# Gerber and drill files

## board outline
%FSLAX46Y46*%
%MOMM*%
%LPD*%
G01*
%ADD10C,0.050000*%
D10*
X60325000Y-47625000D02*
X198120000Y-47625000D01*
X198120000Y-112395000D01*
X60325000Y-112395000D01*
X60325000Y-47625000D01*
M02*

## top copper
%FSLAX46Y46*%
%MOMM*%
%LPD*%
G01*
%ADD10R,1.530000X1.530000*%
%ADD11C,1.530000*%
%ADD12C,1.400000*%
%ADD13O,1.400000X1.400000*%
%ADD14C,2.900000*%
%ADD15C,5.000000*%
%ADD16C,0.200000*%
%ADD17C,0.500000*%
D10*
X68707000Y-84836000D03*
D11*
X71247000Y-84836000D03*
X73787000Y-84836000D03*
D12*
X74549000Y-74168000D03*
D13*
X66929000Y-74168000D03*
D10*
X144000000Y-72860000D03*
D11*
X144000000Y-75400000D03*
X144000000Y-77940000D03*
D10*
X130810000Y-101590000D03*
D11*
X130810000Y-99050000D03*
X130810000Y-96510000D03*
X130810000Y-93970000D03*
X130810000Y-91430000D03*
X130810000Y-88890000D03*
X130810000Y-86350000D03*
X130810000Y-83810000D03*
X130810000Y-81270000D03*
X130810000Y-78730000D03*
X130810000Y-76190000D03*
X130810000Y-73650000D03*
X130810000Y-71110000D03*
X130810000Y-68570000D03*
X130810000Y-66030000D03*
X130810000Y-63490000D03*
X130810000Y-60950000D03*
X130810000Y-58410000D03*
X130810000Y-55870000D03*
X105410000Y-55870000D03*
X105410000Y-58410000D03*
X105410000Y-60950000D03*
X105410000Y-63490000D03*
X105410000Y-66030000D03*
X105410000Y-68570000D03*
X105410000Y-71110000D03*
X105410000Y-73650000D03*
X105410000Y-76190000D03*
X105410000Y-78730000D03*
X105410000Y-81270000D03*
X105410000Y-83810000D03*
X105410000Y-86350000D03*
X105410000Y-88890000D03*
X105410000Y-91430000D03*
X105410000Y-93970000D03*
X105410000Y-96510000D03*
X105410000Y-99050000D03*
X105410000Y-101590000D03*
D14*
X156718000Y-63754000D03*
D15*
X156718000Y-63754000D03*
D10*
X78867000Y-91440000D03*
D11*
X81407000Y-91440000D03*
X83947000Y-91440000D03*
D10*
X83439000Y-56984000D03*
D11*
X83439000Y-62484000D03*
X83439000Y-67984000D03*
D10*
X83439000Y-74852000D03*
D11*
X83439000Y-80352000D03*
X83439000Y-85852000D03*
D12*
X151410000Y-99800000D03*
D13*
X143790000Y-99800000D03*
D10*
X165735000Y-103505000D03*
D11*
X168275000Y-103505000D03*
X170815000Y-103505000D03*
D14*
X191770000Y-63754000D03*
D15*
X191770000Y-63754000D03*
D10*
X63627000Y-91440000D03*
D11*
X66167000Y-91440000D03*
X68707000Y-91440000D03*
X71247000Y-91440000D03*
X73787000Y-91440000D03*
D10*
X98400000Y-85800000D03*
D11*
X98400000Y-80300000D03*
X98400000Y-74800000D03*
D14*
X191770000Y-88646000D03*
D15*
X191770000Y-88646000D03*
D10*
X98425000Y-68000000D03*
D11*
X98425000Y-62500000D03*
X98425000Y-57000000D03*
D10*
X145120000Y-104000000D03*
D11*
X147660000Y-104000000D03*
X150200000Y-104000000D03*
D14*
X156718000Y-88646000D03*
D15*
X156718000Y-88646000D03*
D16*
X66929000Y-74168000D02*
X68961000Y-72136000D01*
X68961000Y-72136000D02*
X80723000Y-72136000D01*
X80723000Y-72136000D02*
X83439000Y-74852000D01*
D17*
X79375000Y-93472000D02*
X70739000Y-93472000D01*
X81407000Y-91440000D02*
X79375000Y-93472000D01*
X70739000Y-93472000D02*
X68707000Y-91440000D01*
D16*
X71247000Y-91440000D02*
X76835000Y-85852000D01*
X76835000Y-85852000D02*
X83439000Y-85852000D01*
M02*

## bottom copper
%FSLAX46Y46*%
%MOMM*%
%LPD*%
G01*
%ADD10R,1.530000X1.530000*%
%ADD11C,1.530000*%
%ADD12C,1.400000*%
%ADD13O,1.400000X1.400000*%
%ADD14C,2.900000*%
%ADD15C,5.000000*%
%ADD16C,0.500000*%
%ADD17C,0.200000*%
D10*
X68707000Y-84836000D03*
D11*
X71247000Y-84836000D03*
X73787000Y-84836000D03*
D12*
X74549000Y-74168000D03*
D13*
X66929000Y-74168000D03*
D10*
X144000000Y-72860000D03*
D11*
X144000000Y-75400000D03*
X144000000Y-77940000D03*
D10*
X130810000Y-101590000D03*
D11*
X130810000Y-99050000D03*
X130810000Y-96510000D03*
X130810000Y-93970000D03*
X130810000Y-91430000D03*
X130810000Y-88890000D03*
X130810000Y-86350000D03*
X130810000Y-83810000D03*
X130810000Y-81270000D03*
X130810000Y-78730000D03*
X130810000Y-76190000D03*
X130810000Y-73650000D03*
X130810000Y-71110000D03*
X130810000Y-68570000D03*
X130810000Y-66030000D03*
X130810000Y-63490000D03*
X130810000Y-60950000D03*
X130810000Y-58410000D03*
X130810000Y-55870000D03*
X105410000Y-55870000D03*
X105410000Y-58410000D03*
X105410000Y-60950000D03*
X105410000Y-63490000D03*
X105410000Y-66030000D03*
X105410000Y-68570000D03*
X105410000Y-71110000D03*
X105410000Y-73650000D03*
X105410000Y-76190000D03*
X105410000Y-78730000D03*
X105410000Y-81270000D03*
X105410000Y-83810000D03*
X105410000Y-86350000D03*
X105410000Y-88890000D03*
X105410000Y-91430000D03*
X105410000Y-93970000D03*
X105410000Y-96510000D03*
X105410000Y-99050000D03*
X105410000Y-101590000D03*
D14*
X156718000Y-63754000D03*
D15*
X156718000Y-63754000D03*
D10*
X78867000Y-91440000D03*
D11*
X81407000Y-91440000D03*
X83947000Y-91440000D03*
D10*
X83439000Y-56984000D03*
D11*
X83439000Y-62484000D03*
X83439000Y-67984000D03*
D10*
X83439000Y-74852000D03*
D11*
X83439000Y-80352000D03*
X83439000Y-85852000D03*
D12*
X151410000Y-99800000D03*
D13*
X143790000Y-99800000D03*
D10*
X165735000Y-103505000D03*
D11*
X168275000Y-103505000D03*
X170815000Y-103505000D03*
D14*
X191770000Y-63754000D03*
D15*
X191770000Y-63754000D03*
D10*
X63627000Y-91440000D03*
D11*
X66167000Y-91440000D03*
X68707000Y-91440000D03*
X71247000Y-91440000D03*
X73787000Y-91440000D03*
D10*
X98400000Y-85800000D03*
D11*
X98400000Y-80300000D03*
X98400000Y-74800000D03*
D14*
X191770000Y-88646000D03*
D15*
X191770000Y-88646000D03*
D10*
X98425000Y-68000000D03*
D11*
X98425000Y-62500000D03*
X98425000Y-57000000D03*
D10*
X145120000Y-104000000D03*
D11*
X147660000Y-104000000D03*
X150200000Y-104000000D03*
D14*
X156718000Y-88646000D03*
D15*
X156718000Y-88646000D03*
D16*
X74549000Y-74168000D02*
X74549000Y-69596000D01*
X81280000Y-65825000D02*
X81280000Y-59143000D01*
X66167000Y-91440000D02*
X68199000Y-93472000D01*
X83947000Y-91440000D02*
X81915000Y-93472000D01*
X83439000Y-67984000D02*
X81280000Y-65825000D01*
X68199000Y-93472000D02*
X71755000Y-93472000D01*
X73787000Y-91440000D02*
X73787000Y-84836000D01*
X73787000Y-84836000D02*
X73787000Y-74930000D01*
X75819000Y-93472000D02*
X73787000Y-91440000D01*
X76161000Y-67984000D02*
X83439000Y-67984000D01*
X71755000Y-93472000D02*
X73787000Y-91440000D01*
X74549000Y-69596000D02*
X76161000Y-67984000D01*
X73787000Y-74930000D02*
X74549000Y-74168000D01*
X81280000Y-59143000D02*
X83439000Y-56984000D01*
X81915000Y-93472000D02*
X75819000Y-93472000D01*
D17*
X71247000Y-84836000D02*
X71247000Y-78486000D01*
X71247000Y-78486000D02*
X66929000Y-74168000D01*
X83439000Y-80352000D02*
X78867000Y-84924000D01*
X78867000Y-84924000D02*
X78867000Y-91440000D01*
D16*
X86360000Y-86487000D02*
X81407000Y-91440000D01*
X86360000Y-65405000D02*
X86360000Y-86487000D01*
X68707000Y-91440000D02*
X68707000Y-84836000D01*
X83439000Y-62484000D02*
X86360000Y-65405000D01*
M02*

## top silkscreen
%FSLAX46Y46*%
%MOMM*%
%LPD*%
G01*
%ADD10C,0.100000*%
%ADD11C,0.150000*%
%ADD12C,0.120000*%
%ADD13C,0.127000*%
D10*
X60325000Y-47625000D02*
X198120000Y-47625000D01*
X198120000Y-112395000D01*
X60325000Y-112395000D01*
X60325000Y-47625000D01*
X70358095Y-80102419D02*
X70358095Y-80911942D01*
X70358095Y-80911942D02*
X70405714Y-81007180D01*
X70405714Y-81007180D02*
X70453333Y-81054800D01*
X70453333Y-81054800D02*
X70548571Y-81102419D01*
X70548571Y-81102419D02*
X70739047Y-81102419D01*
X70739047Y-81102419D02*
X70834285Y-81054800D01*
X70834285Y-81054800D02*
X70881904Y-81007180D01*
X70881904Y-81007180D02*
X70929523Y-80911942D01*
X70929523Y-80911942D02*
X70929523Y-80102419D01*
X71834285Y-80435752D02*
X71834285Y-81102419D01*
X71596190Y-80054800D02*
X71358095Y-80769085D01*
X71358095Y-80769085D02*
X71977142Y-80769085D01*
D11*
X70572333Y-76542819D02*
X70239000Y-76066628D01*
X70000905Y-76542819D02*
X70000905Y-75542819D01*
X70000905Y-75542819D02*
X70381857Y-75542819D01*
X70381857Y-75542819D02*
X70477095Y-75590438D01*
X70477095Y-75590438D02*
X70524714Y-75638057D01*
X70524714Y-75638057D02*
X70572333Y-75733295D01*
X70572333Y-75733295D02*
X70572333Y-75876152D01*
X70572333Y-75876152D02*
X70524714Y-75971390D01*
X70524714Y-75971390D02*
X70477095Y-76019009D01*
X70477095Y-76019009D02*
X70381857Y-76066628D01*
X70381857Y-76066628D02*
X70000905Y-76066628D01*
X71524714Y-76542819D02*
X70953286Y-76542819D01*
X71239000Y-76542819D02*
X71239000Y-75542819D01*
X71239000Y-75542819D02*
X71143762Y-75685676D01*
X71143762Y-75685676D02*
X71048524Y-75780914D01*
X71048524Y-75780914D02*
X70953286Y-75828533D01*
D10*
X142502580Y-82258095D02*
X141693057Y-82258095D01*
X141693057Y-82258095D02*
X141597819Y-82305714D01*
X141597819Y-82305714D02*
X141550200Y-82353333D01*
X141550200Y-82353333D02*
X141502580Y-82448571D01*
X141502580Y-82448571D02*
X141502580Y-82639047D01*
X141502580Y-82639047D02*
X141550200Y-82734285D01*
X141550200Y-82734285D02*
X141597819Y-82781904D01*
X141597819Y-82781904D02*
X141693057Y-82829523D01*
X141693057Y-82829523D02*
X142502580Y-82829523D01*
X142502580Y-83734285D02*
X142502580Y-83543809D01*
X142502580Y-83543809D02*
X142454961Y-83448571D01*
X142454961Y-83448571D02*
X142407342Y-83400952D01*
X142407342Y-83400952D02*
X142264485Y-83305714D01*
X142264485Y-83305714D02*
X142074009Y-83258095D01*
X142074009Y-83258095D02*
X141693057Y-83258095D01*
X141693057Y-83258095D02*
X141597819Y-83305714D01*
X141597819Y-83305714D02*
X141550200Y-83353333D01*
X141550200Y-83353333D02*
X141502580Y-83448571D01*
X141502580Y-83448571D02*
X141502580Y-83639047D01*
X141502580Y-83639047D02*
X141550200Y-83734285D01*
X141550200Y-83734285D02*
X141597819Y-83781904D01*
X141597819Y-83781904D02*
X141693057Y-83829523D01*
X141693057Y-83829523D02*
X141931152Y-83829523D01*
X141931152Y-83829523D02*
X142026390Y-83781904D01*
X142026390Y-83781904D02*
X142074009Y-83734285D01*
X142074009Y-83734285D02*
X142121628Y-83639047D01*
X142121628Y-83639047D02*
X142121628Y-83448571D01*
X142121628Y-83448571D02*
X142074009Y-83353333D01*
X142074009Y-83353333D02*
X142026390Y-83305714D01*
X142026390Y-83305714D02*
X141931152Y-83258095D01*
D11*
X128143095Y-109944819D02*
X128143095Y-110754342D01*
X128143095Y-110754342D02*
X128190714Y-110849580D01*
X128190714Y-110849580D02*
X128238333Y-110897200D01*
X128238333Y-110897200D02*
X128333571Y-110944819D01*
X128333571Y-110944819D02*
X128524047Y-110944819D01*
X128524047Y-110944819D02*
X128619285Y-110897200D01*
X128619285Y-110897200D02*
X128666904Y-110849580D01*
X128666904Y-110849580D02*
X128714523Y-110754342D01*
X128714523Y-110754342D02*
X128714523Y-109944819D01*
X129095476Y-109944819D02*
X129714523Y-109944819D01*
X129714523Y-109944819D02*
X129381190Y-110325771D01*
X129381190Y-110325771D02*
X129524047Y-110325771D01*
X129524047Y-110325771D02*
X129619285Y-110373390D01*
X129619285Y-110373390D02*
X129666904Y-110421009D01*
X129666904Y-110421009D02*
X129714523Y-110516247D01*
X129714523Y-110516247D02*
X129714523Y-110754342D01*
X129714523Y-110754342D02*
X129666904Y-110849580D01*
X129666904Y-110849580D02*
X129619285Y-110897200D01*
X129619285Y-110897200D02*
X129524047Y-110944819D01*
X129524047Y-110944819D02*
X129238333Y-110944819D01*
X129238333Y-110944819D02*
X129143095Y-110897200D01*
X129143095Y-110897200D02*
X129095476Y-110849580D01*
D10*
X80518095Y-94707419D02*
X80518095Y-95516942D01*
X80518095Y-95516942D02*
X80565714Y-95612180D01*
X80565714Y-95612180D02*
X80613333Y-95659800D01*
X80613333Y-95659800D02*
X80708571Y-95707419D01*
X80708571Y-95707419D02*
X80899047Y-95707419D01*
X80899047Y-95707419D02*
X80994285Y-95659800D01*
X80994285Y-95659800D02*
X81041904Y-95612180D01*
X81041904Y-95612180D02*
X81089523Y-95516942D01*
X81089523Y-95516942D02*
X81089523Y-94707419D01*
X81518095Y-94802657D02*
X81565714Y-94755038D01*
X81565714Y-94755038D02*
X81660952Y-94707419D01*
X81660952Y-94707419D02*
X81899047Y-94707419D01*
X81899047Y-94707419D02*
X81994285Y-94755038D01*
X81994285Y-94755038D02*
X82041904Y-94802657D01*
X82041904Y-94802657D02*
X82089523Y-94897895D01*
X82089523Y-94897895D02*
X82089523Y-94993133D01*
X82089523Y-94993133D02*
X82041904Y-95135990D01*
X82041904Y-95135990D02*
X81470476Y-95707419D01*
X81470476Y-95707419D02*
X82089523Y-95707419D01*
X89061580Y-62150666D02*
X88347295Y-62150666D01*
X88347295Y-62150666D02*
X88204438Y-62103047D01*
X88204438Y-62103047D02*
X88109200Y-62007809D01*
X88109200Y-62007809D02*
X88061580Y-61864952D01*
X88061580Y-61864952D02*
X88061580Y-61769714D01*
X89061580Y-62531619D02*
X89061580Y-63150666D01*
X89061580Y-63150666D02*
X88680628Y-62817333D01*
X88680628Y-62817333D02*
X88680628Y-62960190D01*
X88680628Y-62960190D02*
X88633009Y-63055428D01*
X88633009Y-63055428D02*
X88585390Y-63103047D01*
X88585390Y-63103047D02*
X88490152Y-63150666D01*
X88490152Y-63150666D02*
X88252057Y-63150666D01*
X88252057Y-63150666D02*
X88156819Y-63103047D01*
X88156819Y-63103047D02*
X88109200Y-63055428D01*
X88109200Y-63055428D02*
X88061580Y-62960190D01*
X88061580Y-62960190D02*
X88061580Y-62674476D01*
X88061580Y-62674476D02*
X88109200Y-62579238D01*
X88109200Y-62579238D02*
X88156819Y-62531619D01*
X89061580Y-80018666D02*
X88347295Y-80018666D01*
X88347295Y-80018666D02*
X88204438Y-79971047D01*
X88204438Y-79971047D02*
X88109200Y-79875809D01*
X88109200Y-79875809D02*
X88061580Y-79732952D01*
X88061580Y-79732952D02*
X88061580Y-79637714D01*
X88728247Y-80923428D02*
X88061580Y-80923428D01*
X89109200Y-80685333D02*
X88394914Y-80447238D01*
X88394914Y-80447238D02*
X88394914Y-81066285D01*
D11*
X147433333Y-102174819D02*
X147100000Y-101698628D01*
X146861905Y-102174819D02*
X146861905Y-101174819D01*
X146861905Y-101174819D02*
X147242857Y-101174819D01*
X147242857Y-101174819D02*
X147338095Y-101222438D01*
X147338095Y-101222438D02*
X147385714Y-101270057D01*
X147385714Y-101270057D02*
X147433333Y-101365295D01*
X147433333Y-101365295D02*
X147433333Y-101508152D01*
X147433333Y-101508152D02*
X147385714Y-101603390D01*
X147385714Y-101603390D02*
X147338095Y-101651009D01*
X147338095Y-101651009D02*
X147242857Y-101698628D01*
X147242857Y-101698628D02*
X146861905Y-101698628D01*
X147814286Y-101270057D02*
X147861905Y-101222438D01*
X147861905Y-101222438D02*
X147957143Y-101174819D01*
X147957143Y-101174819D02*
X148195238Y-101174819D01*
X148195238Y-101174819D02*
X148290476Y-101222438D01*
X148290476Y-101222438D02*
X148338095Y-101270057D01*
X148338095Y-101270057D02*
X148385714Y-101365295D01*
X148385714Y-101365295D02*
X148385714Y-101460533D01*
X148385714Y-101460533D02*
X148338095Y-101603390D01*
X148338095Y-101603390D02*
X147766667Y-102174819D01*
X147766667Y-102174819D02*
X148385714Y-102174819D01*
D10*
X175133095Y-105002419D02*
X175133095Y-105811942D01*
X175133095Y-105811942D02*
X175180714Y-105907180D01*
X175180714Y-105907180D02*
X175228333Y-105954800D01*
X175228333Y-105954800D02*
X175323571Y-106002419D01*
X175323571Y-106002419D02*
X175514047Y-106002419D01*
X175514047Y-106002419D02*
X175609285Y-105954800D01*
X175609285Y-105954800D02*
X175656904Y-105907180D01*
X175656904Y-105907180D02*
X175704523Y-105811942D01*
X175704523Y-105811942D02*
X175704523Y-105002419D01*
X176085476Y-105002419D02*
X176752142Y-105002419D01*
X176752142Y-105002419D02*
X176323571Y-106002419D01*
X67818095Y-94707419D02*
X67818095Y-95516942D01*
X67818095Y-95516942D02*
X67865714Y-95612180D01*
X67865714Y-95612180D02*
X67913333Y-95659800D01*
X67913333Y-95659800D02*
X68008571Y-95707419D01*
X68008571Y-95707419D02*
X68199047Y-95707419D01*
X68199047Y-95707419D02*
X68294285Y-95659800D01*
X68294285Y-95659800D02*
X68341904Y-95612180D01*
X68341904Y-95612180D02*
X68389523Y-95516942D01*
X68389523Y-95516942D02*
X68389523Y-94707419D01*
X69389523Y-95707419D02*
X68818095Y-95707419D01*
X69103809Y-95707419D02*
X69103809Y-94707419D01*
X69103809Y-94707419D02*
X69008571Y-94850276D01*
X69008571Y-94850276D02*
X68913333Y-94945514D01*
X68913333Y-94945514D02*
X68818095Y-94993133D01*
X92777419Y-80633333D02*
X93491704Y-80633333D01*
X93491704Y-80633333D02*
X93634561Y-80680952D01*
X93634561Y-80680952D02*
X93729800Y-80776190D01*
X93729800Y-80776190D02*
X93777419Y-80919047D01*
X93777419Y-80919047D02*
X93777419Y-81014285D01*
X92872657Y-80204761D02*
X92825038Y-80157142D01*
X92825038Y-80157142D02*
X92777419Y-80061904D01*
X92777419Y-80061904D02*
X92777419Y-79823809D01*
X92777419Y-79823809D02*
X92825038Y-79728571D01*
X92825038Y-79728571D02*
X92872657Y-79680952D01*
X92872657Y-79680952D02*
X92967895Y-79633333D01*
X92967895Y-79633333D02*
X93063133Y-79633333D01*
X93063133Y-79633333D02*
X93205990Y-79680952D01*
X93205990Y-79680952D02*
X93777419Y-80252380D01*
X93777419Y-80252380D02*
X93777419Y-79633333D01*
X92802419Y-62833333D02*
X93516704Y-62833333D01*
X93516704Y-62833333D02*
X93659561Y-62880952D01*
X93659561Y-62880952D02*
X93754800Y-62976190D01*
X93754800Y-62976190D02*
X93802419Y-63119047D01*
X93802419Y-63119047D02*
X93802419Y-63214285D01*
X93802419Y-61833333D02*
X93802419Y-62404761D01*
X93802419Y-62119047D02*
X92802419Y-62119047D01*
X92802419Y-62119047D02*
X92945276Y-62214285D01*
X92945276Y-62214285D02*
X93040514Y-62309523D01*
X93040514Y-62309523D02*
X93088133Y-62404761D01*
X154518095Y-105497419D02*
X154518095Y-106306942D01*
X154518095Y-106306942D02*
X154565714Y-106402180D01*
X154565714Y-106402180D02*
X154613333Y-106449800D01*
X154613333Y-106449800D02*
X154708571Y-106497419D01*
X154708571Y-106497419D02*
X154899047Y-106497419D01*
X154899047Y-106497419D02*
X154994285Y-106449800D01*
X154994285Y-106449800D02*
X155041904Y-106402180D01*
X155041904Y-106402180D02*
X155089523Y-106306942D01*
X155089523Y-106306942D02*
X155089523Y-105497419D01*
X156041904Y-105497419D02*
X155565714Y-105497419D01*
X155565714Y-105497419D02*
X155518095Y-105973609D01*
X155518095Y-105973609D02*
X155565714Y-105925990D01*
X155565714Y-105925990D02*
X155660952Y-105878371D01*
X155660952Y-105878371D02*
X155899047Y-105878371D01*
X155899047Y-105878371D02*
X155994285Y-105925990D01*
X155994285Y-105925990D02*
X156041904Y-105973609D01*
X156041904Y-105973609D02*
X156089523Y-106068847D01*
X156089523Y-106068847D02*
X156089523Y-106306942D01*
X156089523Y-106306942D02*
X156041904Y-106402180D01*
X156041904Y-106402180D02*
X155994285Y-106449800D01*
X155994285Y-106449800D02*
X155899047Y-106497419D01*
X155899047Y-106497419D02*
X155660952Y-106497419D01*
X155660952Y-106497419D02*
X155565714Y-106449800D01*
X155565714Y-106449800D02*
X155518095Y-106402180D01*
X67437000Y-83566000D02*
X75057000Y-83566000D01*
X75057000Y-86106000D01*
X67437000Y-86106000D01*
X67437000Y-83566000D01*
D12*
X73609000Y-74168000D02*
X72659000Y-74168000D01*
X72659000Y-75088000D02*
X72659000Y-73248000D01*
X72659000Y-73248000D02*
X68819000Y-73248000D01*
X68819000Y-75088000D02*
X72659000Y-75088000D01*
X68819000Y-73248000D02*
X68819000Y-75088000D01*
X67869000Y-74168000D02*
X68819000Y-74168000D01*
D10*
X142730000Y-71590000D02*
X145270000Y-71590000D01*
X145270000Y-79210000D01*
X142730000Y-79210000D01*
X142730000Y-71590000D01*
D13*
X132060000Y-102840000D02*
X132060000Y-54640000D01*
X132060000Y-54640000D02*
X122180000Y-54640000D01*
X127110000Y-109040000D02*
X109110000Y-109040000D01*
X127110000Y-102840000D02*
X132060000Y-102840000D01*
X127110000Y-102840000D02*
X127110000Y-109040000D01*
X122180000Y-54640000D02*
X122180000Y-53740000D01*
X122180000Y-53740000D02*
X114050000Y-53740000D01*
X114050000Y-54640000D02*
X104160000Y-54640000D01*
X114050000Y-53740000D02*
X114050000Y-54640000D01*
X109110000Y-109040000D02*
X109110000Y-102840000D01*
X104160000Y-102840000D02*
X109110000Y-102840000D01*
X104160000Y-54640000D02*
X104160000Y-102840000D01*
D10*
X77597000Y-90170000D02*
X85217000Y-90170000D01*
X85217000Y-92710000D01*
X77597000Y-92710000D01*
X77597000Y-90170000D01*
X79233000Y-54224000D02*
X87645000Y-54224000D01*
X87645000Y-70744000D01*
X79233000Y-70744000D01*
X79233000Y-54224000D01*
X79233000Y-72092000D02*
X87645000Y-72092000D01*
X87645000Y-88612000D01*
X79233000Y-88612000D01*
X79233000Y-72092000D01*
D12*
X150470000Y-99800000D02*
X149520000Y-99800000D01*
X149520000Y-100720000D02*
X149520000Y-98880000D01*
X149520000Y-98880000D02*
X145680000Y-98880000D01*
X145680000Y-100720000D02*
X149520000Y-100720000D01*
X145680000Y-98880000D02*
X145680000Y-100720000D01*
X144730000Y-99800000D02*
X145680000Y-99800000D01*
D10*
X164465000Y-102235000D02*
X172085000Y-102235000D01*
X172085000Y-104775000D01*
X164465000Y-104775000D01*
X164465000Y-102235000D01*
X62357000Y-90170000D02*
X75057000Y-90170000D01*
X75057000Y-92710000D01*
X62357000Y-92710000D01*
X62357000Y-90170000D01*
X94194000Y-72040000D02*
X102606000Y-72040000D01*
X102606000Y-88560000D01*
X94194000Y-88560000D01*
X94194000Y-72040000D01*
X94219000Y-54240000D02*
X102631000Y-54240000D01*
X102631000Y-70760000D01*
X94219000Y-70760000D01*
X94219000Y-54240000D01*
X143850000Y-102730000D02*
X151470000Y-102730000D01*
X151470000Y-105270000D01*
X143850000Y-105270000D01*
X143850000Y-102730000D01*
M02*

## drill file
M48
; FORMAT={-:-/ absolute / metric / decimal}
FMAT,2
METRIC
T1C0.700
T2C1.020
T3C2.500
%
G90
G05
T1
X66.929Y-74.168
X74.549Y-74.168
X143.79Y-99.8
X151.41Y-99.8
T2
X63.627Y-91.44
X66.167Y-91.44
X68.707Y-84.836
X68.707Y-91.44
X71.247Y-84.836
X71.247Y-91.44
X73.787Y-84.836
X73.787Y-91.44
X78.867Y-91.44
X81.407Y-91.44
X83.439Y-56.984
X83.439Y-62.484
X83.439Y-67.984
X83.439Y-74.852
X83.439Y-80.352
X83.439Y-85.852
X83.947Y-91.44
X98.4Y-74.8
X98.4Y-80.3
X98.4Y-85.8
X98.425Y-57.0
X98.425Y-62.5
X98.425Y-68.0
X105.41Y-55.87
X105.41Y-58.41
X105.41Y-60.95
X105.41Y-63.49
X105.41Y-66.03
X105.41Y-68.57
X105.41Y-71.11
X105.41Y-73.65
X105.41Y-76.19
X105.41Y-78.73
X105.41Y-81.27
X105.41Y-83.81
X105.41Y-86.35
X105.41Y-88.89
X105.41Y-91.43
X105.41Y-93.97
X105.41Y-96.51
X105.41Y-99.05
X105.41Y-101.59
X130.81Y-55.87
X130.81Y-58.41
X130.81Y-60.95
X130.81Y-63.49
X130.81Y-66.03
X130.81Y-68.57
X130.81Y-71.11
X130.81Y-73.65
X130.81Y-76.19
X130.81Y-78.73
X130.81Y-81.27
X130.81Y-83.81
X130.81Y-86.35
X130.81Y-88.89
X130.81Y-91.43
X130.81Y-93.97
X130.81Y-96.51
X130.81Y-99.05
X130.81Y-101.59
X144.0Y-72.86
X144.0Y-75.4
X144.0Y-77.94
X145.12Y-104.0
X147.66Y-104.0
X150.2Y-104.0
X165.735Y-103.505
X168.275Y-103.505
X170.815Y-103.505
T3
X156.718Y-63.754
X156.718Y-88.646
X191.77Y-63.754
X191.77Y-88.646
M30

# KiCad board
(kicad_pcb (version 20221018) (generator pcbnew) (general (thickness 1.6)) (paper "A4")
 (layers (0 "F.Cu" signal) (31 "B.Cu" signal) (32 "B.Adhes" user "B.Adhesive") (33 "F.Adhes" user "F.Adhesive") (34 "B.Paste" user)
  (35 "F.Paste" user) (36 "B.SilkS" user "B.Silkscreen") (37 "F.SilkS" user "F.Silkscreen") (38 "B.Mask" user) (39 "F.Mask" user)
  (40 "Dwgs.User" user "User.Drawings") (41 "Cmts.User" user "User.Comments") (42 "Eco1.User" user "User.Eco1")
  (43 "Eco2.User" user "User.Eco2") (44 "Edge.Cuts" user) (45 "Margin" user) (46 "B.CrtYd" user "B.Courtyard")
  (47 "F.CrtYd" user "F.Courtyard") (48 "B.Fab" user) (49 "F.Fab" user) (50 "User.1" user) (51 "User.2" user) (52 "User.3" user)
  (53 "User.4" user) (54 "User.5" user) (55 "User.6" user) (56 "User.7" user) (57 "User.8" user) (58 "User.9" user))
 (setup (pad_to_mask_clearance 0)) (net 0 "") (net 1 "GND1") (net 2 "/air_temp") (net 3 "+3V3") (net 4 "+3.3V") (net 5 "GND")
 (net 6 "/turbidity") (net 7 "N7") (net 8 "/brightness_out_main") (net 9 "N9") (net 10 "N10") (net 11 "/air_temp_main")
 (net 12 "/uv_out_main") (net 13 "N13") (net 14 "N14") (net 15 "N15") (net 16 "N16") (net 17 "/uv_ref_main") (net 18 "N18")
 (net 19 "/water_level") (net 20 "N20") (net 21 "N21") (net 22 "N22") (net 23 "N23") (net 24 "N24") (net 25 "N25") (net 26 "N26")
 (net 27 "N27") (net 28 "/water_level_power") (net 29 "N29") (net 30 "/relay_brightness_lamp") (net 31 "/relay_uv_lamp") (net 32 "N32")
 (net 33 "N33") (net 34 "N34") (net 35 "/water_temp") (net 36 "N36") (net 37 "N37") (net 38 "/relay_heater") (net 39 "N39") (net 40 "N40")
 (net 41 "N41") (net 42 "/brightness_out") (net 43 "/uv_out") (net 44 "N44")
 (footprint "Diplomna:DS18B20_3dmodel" (layer "F.Cu") (at 76.327 87.376)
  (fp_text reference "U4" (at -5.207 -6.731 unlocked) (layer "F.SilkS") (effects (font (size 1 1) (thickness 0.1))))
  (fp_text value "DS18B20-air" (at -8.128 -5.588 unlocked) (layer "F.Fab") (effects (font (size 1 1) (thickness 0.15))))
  (fp_rect (start -8.89 -3.81) (end -1.27 -1.27) (stroke (width 0.1) (type default)) (fill none) (layer "F.SilkS"))
  (pad "1" thru_hole rect (at -7.62 -2.54) (size 1.53 1.53) (drill 1.02) (layers "*.Cu" "*.Mask") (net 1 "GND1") (solder_mask_margin 0.102))
  (pad "2" thru_hole circle (at -5.08 -2.54) (size 1.53 1.53) (drill 1.02) (layers "*.Cu" "*.Mask") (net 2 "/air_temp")
   (solder_mask_margin 0.102))
  (pad "3" thru_hole circle (at -2.54 -2.54) (size 1.53 1.53) (drill 1.02) (layers "*.Cu" "*.Mask") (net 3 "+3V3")
   (solder_mask_margin 0.102)))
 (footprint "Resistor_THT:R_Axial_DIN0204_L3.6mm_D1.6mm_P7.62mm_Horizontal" (layer "F.Cu") (at 74.549 74.168 180)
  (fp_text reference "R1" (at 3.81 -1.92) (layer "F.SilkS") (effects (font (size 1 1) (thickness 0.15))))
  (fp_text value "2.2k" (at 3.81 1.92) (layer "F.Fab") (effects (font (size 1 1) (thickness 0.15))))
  (fp_line (start 0.94 0) (end 1.89 0) (stroke (width 0.12) (type solid)) (layer "F.SilkS"))
  (fp_line (start 1.89 -0.92) (end 1.89 0.92) (stroke (width 0.12) (type solid)) (layer "F.SilkS"))
  (fp_line (start 1.89 0.92) (end 5.73 0.92) (stroke (width 0.12) (type solid)) (layer "F.SilkS"))
  (fp_line (start 5.73 -0.92) (end 1.89 -0.92) (stroke (width 0.12) (type solid)) (layer "F.SilkS"))
  (fp_line (start 5.73 0.92) (end 5.73 -0.92) (stroke (width 0.12) (type solid)) (layer "F.SilkS"))
  (fp_line (start 6.68 0) (end 5.73 0) (stroke (width 0.12) (type solid)) (layer "F.SilkS"))
  (pad "1" thru_hole circle (at 0 0 180) (size 1.4 1.4) (drill 0.7) (layers "*.Cu" "*.Mask") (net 3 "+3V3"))
  (pad "2" thru_hole oval (at 7.62 0 180) (size 1.4 1.4) (drill 0.7) (layers "*.Cu" "*.Mask") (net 2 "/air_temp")))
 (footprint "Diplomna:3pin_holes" (layer "F.Cu") (at 141.46 80.48 -90)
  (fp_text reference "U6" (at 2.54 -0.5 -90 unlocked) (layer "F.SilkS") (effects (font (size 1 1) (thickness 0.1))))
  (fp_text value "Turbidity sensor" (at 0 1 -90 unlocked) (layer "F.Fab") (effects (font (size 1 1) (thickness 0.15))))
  (fp_rect (start -8.89 -3.81) (end -1.27 -1.27) (stroke (width 0.1) (type default)) (fill none) (layer "F.SilkS"))
  (pad "1" thru_hole rect (at -7.62 -2.54 270) (size 1.53 1.53) (drill 1.02) (layers "*.Cu" "*.Mask") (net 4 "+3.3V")
   (solder_mask_margin 0.102))
  (pad "2" thru_hole circle (at -5.08 -2.54 270) (size 1.53 1.53) (drill 1.02) (layers "*.Cu" "*.Mask") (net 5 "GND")
   (solder_mask_margin 0.102))
  (pad "3" thru_hole circle (at -2.54 -2.54 270) (size 1.53 1.53) (drill 1.02) (layers "*.Cu" "*.Mask") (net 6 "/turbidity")
   (solder_mask_margin 0.102)))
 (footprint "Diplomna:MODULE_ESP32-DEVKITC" (layer "F.Cu") (at 118.11 78.74 180)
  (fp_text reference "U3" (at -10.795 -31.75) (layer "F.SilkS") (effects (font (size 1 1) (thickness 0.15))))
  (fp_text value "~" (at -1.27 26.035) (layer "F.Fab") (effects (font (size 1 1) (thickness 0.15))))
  (fp_line (start -13.95 -24.1) (end -13.95 24.1) (stroke (width 0.127) (type solid)) (layer "F.SilkS"))
  (fp_line (start -13.95 24.1) (end -4.07 24.1) (stroke (width 0.127) (type solid)) (layer "F.SilkS"))
  (fp_line (start -9 -30.3) (end 9 -30.3) (stroke (width 0.127) (type solid)) (layer "F.SilkS"))
  (fp_line (start -9 -24.1) (end -13.95 -24.1) (stroke (width 0.127) (type solid)) (layer "F.SilkS"))
  (fp_line (start -9 -24.1) (end -9 -30.3) (stroke (width 0.127) (type solid)) (layer "F.SilkS"))
  (fp_line (start -4.07 24.1) (end -4.07 25) (stroke (width 0.127) (type solid)) (layer "F.SilkS"))
  (fp_line (start -4.07 25) (end 4.06 25) (stroke (width 0.127) (type solid)) (layer "F.SilkS"))
  (fp_line (start 4.06 24.1) (end 13.95 24.1) (stroke (width 0.127) (type solid)) (layer "F.SilkS"))
  (fp_line (start 4.06 25) (end 4.06 24.1) (stroke (width 0.127) (type solid)) (layer "F.SilkS"))
  (fp_line (start 9 -30.3) (end 9 -24.1) (stroke (width 0.127) (type solid)) (layer "F.SilkS"))
  (fp_line (start 13.95 -24.1) (end 9 -24.1) (stroke (width 0.127) (type solid)) (layer "F.SilkS"))
  (fp_line (start 13.95 24.1) (end 13.95 -24.1) (stroke (width 0.127) (type solid)) (layer "F.SilkS"))
  (pad "1" thru_hole rect (at -12.7 -22.85 180) (size 1.53 1.53) (drill 1.02) (layers "*.Cu" "*.Mask") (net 4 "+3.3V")
   (solder_mask_margin 0.102))
  (pad "2" thru_hole circle (at -12.7 -20.31 180) (size 1.53 1.53) (drill 1.02) (layers "*.Cu" "*.Mask") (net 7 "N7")
   (solder_mask_margin 0.102))
  (pad "3" thru_hole circle (at -12.7 -17.77 180) (size 1.53 1.53) (drill 1.02) (layers "*.Cu" "*.Mask") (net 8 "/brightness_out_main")
   (solder_mask_margin 0.102))
  (pad "4" thru_hole circle (at -12.7 -15.23 180) (size 1.53 1.53) (drill 1.02) (layers "*.Cu" "*.Mask") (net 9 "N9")
   (solder_mask_margin 0.102))
  (pad "5" thru_hole circle (at -12.7 -12.69 180) (size 1.53 1.53) (drill 1.02) (layers "*.Cu" "*.Mask") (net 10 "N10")
   (solder_mask_margin 0.102))
  (pad "6" thru_hole circle (at -12.7 -10.15 180) (size 1.53 1.53) (drill 1.02) (layers "*.Cu" "*.Mask") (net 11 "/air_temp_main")
   (solder_mask_margin 0.102))
  (pad "7" thru_hole circle (at -12.7 -7.61 180) (size 1.53 1.53) (drill 1.02) (layers "*.Cu" "*.Mask") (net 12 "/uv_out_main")
   (solder_mask_margin 0.102))
  (pad "8" thru_hole circle (at -12.7 -5.07 180) (size 1.53 1.53) (drill 1.02) (layers "*.Cu" "*.Mask") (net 6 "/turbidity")
   (solder_mask_margin 0.102))
  (pad "9" thru_hole circle (at -12.7 -2.53 180) (size 1.53 1.53) (drill 1.02) (layers "*.Cu" "*.Mask") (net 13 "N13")
   (solder_mask_margin 0.102))
  (pad "10" thru_hole circle (at -12.7 0.01 180) (size 1.53 1.53) (drill 1.02) (layers "*.Cu" "*.Mask") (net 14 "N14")
   (solder_mask_margin 0.102))
  (pad "11" thru_hole circle (at -12.7 2.55 180) (size 1.53 1.53) (drill 1.02) (layers "*.Cu" "*.Mask") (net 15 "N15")
   (solder_mask_margin 0.102))
  (pad "12" thru_hole circle (at -12.7 5.09 180) (size 1.53 1.53) (drill 1.02) (layers "*.Cu" "*.Mask") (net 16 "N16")
   (solder_mask_margin 0.102))
  (pad "13" thru_hole circle (at -12.7 7.63 180) (size 1.53 1.53) (drill 1.02) (layers "*.Cu" "*.Mask") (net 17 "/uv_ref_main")
   (solder_mask_margin 0.102))
  (pad "14" thru_hole circle (at -12.7 10.17 180) (size 1.53 1.53) (drill 1.02) (layers "*.Cu" "*.Mask") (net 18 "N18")
   (solder_mask_margin 0.102))
  (pad "15" thru_hole circle (at -12.7 12.71 180) (size 1.53 1.53) (drill 1.02) (layers "*.Cu" "*.Mask") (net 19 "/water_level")
   (solder_mask_margin 0.102))
  (pad "16" thru_hole circle (at -12.7 15.25 180) (size 1.53 1.53) (drill 1.02) (layers "*.Cu" "*.Mask") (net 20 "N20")
   (solder_mask_margin 0.102))
  (pad "17" thru_hole circle (at -12.7 17.79 180) (size 1.53 1.53) (drill 1.02) (layers "*.Cu" "*.Mask") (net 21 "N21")
   (solder_mask_margin 0.102))
  (pad "18" thru_hole circle (at -12.7 20.33 180) (size 1.53 1.53) (drill 1.02) (layers "*.Cu" "*.Mask") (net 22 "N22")
   (solder_mask_margin 0.102))
  (pad "19" thru_hole circle (at -12.7 22.87 180) (size 1.53 1.53) (drill 1.02) (layers "*.Cu" "*.Mask") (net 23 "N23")
   (solder_mask_margin 0.102))
  (pad "20" thru_hole circle (at 12.7 22.87 180) (size 1.53 1.53) (drill 1.02) (layers "*.Cu" "*.Mask") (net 5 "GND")
   (solder_mask_margin 0.102))
  (pad "21" thru_hole circle (at 12.7 20.33 180) (size 1.53 1.53) (drill 1.02) (layers "*.Cu" "*.Mask") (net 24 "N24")
   (solder_mask_margin 0.102))
  (pad "22" thru_hole circle (at 12.7 17.79 180) (size 1.53 1.53) (drill 1.02) (layers "*.Cu" "*.Mask") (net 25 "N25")
   (solder_mask_margin 0.102))
  (pad "23" thru_hole circle (at 12.7 15.25 180) (size 1.53 1.53) (drill 1.02) (layers "*.Cu" "*.Mask") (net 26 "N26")
   (solder_mask_margin 0.102))
  (pad "24" thru_hole circle (at 12.7 12.71 180) (size 1.53 1.53) (drill 1.02) (layers "*.Cu" "*.Mask") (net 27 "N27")
   (solder_mask_margin 0.102))
  (pad "25" thru_hole circle (at 12.7 10.17 180) (size 1.53 1.53) (drill 1.02) (layers "*.Cu" "*.Mask") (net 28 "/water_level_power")
   (solder_mask_margin 0.102))
  (pad "26" thru_hole circle (at 12.7 7.63 180) (size 1.53 1.53) (drill 1.02) (layers "*.Cu" "*.Mask") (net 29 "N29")
   (solder_mask_margin 0.102))
  (pad "27" thru_hole circle (at 12.7 5.09 180) (size 1.53 1.53) (drill 1.02) (layers "*.Cu" "*.Mask") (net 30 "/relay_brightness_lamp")
   (solder_mask_margin 0.102))
  (pad "28" thru_hole circle (at 12.7 2.55 180) (size 1.53 1.53) (drill 1.02) (layers "*.Cu" "*.Mask") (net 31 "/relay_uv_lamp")
   (solder_mask_margin 0.102))
  (pad "29" thru_hole circle (at 12.7 0.01 180) (size 1.53 1.53) (drill 1.02) (layers "*.Cu" "*.Mask") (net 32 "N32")
   (solder_mask_margin 0.102))
  (pad "30" thru_hole circle (at 12.7 -2.53 180) (size 1.53 1.53) (drill 1.02) (layers "*.Cu" "*.Mask") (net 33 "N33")
   (solder_mask_margin 0.102))
  (pad "31" thru_hole circle (at 12.7 -5.07 180) (size 1.53 1.53) (drill 1.02) (layers "*.Cu" "*.Mask") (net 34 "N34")
   (solder_mask_margin 0.102))
  (pad "32" thru_hole circle (at 12.7 -7.61 180) (size 1.53 1.53) (drill 1.02) (layers "*.Cu" "*.Mask") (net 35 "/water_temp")
   (solder_mask_margin 0.102))
  (pad "33" thru_hole circle (at 12.7 -10.15 180) (size 1.53 1.53) (drill 1.02) (layers "*.Cu" "*.Mask") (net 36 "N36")
   (solder_mask_margin 0.102))
  (pad "34" thru_hole circle (at 12.7 -12.69 180) (size 1.53 1.53) (drill 1.02) (layers "*.Cu" "*.Mask") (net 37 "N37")
   (solder_mask_margin 0.102))
  (pad "35" thru_hole circle (at 12.7 -15.23 180) (size 1.53 1.53) (drill 1.02) (layers "*.Cu" "*.Mask") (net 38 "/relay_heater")
   (solder_mask_margin 0.102))
  (pad "36" thru_hole circle (at 12.7 -17.77 180) (size 1.53 1.53) (drill 1.02) (layers "*.Cu" "*.Mask") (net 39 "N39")
   (solder_mask_margin 0.102))
  (pad "37" thru_hole circle (at 12.7 -20.31 180) (size 1.53 1.53) (drill 1.02) (layers "*.Cu" "*.Mask") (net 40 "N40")
   (solder_mask_margin 0.102))
  (pad "38" thru_hole circle (at 12.7 -22.85 180) (size 1.53 1.53) (drill 1.02) (layers "*.Cu" "*.Mask") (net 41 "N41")
   (solder_mask_margin 0.102)))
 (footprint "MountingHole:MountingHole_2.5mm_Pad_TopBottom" (layer "F.Cu") (at 156.718 63.754)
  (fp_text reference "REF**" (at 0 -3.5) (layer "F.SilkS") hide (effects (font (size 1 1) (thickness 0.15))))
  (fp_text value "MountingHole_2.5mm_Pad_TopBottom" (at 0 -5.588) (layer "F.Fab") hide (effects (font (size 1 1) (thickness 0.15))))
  (pad "1" thru_hole circle (at 0 0) (size 2.9 2.9) (drill 2.5) (layers "*.Cu" "*.Mask"))
  (pad "1" connect circle (at 0 0) (size 5 5) (layers "F.Cu" "F.Mask"))
  (pad "1" connect circle (at 0 0) (size 5 5) (layers "B.Cu" "B.Mask")))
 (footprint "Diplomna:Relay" (layer "F.Cu") (at 254.508 101.092 -90)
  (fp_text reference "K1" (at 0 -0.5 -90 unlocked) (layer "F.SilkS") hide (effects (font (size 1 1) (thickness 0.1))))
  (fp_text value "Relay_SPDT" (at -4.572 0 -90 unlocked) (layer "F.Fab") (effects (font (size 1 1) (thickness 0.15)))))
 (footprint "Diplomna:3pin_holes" (layer "F.Cu") (at 86.487 93.98)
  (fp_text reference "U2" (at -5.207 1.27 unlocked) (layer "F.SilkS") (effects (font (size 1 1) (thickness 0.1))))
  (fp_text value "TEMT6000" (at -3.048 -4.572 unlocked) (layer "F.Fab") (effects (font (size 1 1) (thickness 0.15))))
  (fp_rect (start -8.89 -3.81) (end -1.27 -1.27) (stroke (width 0.1) (type default)) (fill none) (layer "F.SilkS"))
  (pad "1" thru_hole rect (at -7.62 -2.54) (size 1.53 1.53) (drill 1.02) (layers "*.Cu" "*.Mask") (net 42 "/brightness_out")
   (solder_mask_margin 0.102))
  (pad "2" thru_hole circle (at -5.08 -2.54) (size 1.53 1.53) (drill 1.02) (layers "*.Cu" "*.Mask") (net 1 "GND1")
   (solder_mask_margin 0.102))
  (pad "3" thru_hole circle (at -2.54 -2.54) (size 1.53 1.53) (drill 1.02) (layers "*.Cu" "*.Mask") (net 3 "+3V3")
   (solder_mask_margin 0.102)))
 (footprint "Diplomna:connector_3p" (layer "F.Cu") (at 83.439 62.484 -90)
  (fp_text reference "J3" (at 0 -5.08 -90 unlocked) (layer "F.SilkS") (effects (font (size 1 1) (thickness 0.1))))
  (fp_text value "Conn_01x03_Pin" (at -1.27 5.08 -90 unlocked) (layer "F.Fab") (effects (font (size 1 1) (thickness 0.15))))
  (fp_rect (start -8.26 -4.206) (end 8.26 4.206) (stroke (width 0.1) (type default)) (fill none) (layer "F.SilkS"))
  (pad "1" thru_hole rect (at -5.5 0 270) (size 1.53 1.53) (drill 1.02) (layers "*.Cu" "*.Mask") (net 3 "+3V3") (solder_mask_margin 0.102))
  (pad "2" thru_hole circle (at 0 0 270) (size 1.53 1.53) (drill 1.02) (layers "*.Cu" "*.Mask") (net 1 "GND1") (solder_mask_margin 0.102))
  (pad "3" thru_hole circle (at 5.5 0 270) (size 1.53 1.53) (drill 1.02) (layers "*.Cu" "*.Mask") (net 3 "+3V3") (solder_mask_margin 0.102)))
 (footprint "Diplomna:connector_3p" (layer "F.Cu") (at 83.439 80.352 -90)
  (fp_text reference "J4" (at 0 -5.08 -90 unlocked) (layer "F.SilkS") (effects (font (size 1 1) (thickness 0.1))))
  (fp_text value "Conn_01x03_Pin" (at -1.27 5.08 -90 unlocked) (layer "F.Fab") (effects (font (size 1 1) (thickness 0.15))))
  (fp_rect (start -8.26 -4.206) (end 8.26 4.206) (stroke (width 0.1) (type default)) (fill none) (layer "F.SilkS"))
  (pad "1" thru_hole rect (at -5.5 0 270) (size 1.53 1.53) (drill 1.02) (layers "*.Cu" "*.Mask") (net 2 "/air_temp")
   (solder_mask_margin 0.102))
  (pad "2" thru_hole circle (at 0 0 270) (size 1.53 1.53) (drill 1.02) (layers "*.Cu" "*.Mask") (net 42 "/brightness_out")
   (solder_mask_margin 0.102))
  (pad "3" thru_hole circle (at 5.5 0 270) (size 1.53 1.53) (drill 1.02) (layers "*.Cu" "*.Mask") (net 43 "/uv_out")
   (solder_mask_margin 0.102)))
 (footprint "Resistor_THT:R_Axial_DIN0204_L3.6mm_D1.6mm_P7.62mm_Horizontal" (layer "F.Cu") (at 151.41 99.8 180)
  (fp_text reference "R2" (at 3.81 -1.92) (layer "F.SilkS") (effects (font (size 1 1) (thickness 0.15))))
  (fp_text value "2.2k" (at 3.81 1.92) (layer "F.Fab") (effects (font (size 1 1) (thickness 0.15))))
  (fp_line (start 0.94 0) (end 1.89 0) (stroke (width 0.12) (type solid)) (layer "F.SilkS"))
  (fp_line (start 1.89 -0.92) (end 1.89 0.92) (stroke (width 0.12) (type solid)) (layer "F.SilkS"))
  (fp_line (start 1.89 0.92) (end 5.73 0.92) (stroke (width 0.12) (type solid)) (layer "F.SilkS"))
  (fp_line (start 5.73 -0.92) (end 1.89 -0.92) (stroke (width 0.12) (type solid)) (layer "F.SilkS"))
  (fp_line (start 5.73 0.92) (end 5.73 -0.92) (stroke (width 0.12) (type solid)) (layer "F.SilkS"))
  (fp_line (start 6.68 0) (end 5.73 0) (stroke (width 0.12) (type solid)) (layer "F.SilkS"))
  (pad "1" thru_hole circle (at 0 0 180) (size 1.4 1.4) (drill 0.7) (layers "*.Cu" "*.Mask") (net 4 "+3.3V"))
  (pad "2" thru_hole oval (at 7.62 0 180) (size 1.4 1.4) (drill 0.7) (layers "*.Cu" "*.Mask") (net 35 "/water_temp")))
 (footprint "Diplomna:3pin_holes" (layer "F.Cu") (at 173.355 106.045)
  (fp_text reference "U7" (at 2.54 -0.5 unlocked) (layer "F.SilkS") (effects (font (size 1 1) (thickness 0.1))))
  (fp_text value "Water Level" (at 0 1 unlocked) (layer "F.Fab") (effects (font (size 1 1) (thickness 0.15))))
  (fp_rect (start -8.89 -3.81) (end -1.27 -1.27) (stroke (width 0.1) (type default)) (fill none) (layer "F.SilkS"))
  (pad "1" thru_hole rect (at -7.62 -2.54) (size 1.53 1.53) (drill 1.02) (layers "*.Cu" "*.Mask") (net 5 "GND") (solder_mask_margin 0.102))
  (pad "2" thru_hole circle (at -5.08 -2.54) (size 1.53 1.53) (drill 1.02) (layers "*.Cu" "*.Mask") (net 28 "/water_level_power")
   (solder_mask_margin 0.102))
  (pad "3" thru_hole circle (at -2.54 -2.54) (size 1.53 1.53) (drill 1.02) (layers "*.Cu" "*.Mask") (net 19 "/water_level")
   (solder_mask_margin 0.102)))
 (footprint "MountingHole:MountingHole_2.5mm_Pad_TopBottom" (layer "F.Cu") (at 191.77 63.754)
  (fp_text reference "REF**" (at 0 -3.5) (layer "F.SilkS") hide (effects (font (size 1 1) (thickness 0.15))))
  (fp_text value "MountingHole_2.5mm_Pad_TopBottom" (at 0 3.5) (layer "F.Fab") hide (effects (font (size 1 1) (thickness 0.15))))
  (pad "1" thru_hole circle (at 0 0) (size 2.9 2.9) (drill 2.5) (layers "*.Cu" "*.Mask"))
  (pad "1" connect circle (at 0 0) (size 5 5) (layers "F.Cu" "F.Mask"))
  (pad "1" connect circle (at 0 0) (size 5 5) (layers "B.Cu" "B.Mask")))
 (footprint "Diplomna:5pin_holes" (layer "F.Cu") (at 78.867 97.155)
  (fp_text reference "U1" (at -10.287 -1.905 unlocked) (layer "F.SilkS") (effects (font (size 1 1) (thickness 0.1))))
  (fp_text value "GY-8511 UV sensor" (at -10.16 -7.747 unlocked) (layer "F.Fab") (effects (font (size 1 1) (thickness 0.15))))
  (fp_rect (start -16.51 -6.985) (end -3.81 -4.445) (stroke (width 0.1) (type default)) (fill none) (layer "F.SilkS"))
  (pad "1" thru_hole rect (at -15.24 -5.715) (size 1.53 1.53) (drill 1.02) (layers "*.Cu" "*.Mask") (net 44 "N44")
   (solder_mask_margin 0.102))
  (pad "2" thru_hole circle (at -12.7 -5.715) (size 1.53 1.53) (drill 1.02) (layers "*.Cu" "*.Mask") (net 3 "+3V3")
   (solder_mask_margin 0.102))
  (pad "3" thru_hole circle (at -10.16 -5.715) (size 1.53 1.53) (drill 1.02) (layers "*.Cu" "*.Mask") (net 1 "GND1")
   (solder_mask_margin 0.102))
  (pad "4" thru_hole circle (at -7.62 -5.715) (size 1.53 1.53) (drill 1.02) (layers "*.Cu" "*.Mask") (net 43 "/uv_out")
   (solder_mask_margin 0.102))
  (pad "5" thru_hole circle (at -5.08 -5.715) (size 1.53 1.53) (drill 1.02) (layers "*.Cu" "*.Mask") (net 3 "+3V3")
   (solder_mask_margin 0.102)))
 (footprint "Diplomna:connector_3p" (layer "F.Cu") (at 98.4 80.3 90)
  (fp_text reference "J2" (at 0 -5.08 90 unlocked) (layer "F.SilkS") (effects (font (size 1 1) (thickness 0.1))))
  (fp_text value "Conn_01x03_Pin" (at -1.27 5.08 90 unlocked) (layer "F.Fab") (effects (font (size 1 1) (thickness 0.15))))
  (fp_rect (start -8.26 -4.206) (end 8.26 4.206) (stroke (width 0.1) (type default)) (fill none) (layer "F.SilkS"))
  (pad "1" thru_hole rect (at -5.5 0 90) (size 1.53 1.53) (drill 1.02) (layers "*.Cu" "*.Mask") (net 11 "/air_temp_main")
   (solder_mask_margin 0.102))
  (pad "2" thru_hole circle (at 0 0 90) (size 1.53 1.53) (drill 1.02) (layers "*.Cu" "*.Mask") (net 8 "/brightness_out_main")
   (solder_mask_margin 0.102))
  (pad "3" thru_hole circle (at 5.5 0 90) (size 1.53 1.53) (drill 1.02) (layers "*.Cu" "*.Mask") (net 12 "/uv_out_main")
   (solder_mask_margin 0.102)))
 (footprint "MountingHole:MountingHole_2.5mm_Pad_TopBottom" (layer "F.Cu") (at 191.77 88.646)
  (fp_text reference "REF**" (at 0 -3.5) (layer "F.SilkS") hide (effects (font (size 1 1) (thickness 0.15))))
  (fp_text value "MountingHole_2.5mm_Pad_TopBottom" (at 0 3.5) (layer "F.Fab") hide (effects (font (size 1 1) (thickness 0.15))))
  (pad "1" thru_hole circle (at 0 0) (size 2.9 2.9) (drill 2.5) (layers "*.Cu" "*.Mask"))
  (pad "1" connect circle (at 0 0) (size 5 5) (layers "F.Cu" "F.Mask"))
  (pad "1" connect circle (at 0 0) (size 5 5) (layers "B.Cu" "B.Mask")))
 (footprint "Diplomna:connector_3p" (layer "F.Cu") (at 98.425 62.5 90)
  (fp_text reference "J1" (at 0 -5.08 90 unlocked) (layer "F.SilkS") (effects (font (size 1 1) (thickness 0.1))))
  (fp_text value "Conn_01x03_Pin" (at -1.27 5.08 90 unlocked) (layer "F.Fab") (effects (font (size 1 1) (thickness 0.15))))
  (fp_rect (start -8.26 -4.206) (end 8.26 4.206) (stroke (width 0.1) (type default)) (fill none) (layer "F.SilkS"))
  (pad "1" thru_hole rect (at -5.5 0 90) (size 1.53 1.53) (drill 1.02) (layers "*.Cu" "*.Mask") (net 4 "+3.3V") (solder_mask_margin 0.102))
  (pad "2" thru_hole circle (at 0 0 90) (size 1.53 1.53) (drill 1.02) (layers "*.Cu" "*.Mask") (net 5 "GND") (solder_mask_margin 0.102))
  (pad "3" thru_hole circle (at 5.5 0 90) (size 1.53 1.53) (drill 1.02) (layers "*.Cu" "*.Mask") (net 17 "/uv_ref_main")
   (solder_mask_margin 0.102)))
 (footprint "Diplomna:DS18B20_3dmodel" (layer "F.Cu") (at 152.74 106.54)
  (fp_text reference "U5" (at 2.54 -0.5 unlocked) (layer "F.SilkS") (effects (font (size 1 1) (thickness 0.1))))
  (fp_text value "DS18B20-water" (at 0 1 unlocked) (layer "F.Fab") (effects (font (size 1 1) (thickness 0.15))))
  (fp_rect (start -8.89 -3.81) (end -1.27 -1.27) (stroke (width 0.1) (type default)) (fill none) (layer "F.SilkS"))
  (pad "1" thru_hole rect (at -7.62 -2.54) (size 1.53 1.53) (drill 1.02) (layers "*.Cu" "*.Mask") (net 5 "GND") (solder_mask_margin 0.102))
  (pad "2" thru_hole circle (at -5.08 -2.54) (size 1.53 1.53) (drill 1.02) (layers "*.Cu" "*.Mask") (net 35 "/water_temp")
   (solder_mask_margin 0.102))
  (pad "3" thru_hole circle (at -2.54 -2.54) (size 1.53 1.53) (drill 1.02) (layers "*.Cu" "*.Mask") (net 4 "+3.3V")
   (solder_mask_margin 0.102)))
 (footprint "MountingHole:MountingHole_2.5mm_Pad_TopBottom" (layer "F.Cu") (at 156.718 88.646)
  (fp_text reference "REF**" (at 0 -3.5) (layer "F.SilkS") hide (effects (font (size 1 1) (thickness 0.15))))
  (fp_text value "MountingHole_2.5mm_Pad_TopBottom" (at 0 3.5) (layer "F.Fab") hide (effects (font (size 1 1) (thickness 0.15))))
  (pad "1" thru_hole circle (at 0 0) (size 2.9 2.9) (drill 2.5) (layers "*.Cu" "*.Mask"))
  (pad "1" connect circle (at 0 0) (size 5 5) (layers "F.Cu" "F.Mask"))
  (pad "1" connect circle (at 0 0) (size 5 5) (layers "B.Cu" "B.Mask")))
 (gr_rect (start 60.325 47.625) (end 198.12 112.395) (stroke (width 0.1) (type default)) (fill none) (layer "F.SilkS"))
 (gr_rect (start 60.325 47.625) (end 198.12 112.395) (stroke (width 0.05) (type default)) (fill none) (layer "Edge.Cuts"))
 (segment (start 74.549 74.168) (end 74.549 69.596) (width 0.5) (layer "B.Cu") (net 3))
 (segment (start 81.28 65.825) (end 81.28 59.143) (width 0.5) (layer "B.Cu") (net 3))
 (segment (start 66.167 91.44) (end 68.199 93.472) (width 0.5) (layer "B.Cu") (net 3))
 (segment (start 83.947 91.44) (end 81.915 93.472) (width 0.5) (layer "B.Cu") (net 3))
 (segment (start 83.439 67.984) (end 81.28 65.825) (width 0.5) (layer "B.Cu") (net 3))
 (segment (start 68.199 93.472) (end 71.755 93.472) (width 0.5) (layer "B.Cu") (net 3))
 (segment (start 73.787 91.44) (end 73.787 84.836) (width 0.5) (layer "B.Cu") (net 3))
 (segment (start 73.787 84.836) (end 73.787 74.93) (width 0.5) (layer "B.Cu") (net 3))
 (segment (start 75.819 93.472) (end 73.787 91.44) (width 0.5) (layer "B.Cu") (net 3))
 (segment (start 76.161 67.984) (end 83.439 67.984) (width 0.5) (layer "B.Cu") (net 3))
 (segment (start 71.755 93.472) (end 73.787 91.44) (width 0.5) (layer "B.Cu") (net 3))
 (segment (start 74.549 69.596) (end 76.161 67.984) (width 0.5) (layer "B.Cu") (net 3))
 (segment (start 73.787 74.93) (end 74.549 74.168) (width 0.5) (layer "B.Cu") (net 3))
 (segment (start 81.28 59.143) (end 83.439 56.984) (width 0.5) (layer "B.Cu") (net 3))
 (segment (start 81.915 93.472) (end 75.819 93.472) (width 0.5) (layer "B.Cu") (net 3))
 (segment (start 66.929 74.168) (end 68.961 72.136) (width 0.2) (layer "F.Cu") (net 2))
 (segment (start 68.961 72.136) (end 80.723 72.136) (width 0.2) (layer "F.Cu") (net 2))
 (segment (start 80.723 72.136) (end 83.439 74.852) (width 0.2) (layer "F.Cu") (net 2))
 (segment (start 71.247 84.836) (end 71.247 78.486) (width 0.2) (layer "B.Cu") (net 2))
 (segment (start 71.247 78.486) (end 66.929 74.168) (width 0.2) (layer "B.Cu") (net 2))
 (segment (start 83.439 80.352) (end 78.867 84.924) (width 0.2) (layer "B.Cu") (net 42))
 (segment (start 78.867 84.924) (end 78.867 91.44) (width 0.2) (layer "B.Cu") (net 42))
 (segment (start 79.375 93.472) (end 70.739 93.472) (width 0.5) (layer "F.Cu") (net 1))
 (segment (start 81.407 91.44) (end 79.375 93.472) (width 0.5) (layer "F.Cu") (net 1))
 (segment (start 70.739 93.472) (end 68.707 91.44) (width 0.5) (layer "F.Cu") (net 1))
 (segment (start 86.36 86.487) (end 81.407 91.44) (width 0.5) (layer "B.Cu") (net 1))
 (segment (start 86.36 65.405) (end 86.36 86.487) (width 0.5) (layer "B.Cu") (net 1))
 (segment (start 68.707 91.44) (end 68.707 84.836) (width 0.5) (layer "B.Cu") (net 1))
 (segment (start 83.439 62.484) (end 86.36 65.405) (width 0.5) (layer "B.Cu") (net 1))
 (segment (start 71.247 91.44) (end 76.835 85.852) (width 0.2) (layer "F.Cu") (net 43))
 (segment (start 76.835 85.852) (end 83.439 85.852) (width 0.2) (layer "F.Cu") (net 43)))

